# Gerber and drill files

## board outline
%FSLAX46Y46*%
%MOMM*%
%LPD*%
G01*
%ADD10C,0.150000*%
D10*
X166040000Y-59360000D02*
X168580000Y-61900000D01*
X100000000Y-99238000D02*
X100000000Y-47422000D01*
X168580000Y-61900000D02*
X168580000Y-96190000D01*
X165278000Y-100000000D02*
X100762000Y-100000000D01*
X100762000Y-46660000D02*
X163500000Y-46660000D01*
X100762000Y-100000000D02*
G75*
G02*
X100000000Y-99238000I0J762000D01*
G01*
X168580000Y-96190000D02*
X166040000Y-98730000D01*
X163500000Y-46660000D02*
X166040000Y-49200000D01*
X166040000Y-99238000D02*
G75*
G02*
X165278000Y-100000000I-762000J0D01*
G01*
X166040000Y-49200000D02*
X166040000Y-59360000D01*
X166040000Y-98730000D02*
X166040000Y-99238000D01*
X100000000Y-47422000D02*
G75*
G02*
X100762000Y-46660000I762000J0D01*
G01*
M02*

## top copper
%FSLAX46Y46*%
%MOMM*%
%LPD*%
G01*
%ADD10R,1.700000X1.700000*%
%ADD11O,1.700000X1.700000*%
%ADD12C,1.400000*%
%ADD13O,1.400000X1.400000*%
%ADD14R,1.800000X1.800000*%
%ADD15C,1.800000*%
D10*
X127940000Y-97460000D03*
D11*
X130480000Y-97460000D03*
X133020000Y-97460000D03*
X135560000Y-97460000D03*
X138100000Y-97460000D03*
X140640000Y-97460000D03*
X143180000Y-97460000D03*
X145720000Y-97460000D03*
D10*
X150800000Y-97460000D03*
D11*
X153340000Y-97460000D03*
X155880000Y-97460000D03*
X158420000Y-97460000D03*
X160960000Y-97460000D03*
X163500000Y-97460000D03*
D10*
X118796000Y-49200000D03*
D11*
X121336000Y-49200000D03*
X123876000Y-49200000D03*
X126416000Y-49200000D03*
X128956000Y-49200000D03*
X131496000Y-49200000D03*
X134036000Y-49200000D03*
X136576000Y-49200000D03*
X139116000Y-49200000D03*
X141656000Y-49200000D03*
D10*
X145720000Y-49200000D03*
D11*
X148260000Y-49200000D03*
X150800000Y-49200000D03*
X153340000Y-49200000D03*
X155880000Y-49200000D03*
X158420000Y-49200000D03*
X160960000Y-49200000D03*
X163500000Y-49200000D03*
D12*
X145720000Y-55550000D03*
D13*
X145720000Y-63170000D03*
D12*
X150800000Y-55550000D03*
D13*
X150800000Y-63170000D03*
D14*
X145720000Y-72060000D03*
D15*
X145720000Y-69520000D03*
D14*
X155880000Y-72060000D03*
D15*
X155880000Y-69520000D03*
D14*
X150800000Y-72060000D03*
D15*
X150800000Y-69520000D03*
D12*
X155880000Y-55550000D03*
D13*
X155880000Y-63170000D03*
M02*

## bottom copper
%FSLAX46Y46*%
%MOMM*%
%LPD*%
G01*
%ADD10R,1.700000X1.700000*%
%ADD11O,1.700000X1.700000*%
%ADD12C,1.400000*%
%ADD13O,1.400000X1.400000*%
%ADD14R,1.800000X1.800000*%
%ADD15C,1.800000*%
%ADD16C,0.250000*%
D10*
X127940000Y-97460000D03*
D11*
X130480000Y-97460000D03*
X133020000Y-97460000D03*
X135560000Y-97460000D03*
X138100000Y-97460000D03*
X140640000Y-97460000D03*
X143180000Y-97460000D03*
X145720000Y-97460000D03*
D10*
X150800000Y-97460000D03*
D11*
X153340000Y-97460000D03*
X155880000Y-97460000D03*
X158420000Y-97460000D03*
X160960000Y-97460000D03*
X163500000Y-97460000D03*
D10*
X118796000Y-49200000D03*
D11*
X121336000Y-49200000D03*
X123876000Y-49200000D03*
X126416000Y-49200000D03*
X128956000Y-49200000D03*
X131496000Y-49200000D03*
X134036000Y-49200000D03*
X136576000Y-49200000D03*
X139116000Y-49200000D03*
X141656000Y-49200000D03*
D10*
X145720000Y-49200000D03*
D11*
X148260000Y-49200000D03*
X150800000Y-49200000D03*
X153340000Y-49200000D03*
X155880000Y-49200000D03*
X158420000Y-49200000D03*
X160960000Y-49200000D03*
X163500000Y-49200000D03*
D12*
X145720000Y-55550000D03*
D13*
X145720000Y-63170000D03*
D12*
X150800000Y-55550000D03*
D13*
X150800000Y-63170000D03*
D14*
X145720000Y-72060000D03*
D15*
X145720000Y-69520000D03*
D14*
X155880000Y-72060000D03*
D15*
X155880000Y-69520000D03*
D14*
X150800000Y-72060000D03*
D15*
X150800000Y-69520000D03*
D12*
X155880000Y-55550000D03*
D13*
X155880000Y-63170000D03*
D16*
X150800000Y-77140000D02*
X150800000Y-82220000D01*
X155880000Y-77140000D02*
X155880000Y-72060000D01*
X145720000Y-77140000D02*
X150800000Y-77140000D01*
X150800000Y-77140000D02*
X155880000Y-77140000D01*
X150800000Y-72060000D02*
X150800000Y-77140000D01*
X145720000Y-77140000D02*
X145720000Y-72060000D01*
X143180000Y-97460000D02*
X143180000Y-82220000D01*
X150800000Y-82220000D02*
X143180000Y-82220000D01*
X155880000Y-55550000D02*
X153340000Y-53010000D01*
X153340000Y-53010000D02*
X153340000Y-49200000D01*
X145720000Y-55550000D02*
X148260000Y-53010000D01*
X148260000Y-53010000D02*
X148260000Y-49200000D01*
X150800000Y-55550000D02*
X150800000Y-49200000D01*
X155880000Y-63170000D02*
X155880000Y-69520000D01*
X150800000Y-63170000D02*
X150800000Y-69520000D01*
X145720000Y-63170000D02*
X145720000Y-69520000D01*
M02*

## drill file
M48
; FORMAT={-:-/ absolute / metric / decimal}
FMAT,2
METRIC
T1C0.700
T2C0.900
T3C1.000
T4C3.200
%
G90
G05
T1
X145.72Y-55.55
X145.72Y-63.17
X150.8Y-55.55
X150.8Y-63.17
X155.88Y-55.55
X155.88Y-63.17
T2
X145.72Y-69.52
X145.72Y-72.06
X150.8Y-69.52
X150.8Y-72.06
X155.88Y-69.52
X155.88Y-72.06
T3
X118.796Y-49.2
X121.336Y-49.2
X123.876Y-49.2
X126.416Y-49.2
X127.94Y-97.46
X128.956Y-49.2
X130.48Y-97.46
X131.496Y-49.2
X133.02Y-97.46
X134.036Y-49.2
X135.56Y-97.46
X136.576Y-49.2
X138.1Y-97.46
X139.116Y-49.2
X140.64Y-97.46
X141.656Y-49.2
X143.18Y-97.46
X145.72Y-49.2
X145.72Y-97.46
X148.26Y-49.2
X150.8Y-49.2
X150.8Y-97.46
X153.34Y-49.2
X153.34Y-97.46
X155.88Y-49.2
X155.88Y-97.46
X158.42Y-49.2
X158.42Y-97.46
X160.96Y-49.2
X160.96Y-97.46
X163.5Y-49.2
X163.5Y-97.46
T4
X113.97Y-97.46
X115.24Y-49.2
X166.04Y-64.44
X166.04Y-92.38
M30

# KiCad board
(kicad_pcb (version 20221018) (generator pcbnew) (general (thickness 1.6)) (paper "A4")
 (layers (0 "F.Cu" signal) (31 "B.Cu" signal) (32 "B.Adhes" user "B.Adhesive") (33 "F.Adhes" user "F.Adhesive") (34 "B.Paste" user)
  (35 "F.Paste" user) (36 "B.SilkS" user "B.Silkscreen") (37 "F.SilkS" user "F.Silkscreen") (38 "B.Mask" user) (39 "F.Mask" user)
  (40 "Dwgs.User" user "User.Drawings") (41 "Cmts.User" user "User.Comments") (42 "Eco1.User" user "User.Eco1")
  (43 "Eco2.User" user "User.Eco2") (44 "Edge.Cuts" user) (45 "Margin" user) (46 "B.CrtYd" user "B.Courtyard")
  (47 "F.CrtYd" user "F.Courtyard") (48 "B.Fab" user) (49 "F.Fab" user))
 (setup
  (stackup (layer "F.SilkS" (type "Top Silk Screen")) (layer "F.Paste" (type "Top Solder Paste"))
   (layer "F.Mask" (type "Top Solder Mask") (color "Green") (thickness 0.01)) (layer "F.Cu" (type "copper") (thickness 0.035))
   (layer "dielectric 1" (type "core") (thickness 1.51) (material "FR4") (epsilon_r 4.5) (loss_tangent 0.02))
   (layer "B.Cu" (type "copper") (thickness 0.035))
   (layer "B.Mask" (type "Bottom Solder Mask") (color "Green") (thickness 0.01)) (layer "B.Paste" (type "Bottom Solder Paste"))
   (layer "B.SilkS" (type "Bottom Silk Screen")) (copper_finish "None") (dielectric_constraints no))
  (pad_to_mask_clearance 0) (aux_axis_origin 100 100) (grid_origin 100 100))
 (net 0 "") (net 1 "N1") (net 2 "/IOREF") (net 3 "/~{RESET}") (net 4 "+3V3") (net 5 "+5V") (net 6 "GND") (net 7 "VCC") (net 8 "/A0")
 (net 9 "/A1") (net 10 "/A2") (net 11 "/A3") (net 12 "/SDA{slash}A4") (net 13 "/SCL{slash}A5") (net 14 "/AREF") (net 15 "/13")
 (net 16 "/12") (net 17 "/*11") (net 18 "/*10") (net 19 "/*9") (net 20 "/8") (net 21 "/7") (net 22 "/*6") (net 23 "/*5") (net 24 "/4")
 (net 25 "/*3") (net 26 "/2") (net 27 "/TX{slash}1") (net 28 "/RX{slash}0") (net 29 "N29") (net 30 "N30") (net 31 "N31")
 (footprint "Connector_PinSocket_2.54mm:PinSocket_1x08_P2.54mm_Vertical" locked (layer "F.Cu") (at 127.94 97.46 90)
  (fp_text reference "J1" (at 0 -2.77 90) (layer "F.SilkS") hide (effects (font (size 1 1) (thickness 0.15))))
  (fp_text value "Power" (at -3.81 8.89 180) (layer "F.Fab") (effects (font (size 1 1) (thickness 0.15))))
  (pad "1" thru_hole rect locked (at 0 0 90) (size 1.7 1.7) (drill 1) (layers "*.Cu" "*.Mask") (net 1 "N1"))
  (pad "2" thru_hole oval locked (at 0 2.54 90) (size 1.7 1.7) (drill 1) (layers "*.Cu" "*.Mask") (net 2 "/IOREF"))
  (pad "3" thru_hole oval locked (at 0 5.08 90) (size 1.7 1.7) (drill 1) (layers "*.Cu" "*.Mask") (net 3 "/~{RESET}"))
  (pad "4" thru_hole oval locked (at 0 7.62 90) (size 1.7 1.7) (drill 1) (layers "*.Cu" "*.Mask") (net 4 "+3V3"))
  (pad "5" thru_hole oval locked (at 0 10.16 90) (size 1.7 1.7) (drill 1) (layers "*.Cu" "*.Mask") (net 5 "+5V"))
  (pad "6" thru_hole oval locked (at 0 12.7 90) (size 1.7 1.7) (drill 1) (layers "*.Cu" "*.Mask") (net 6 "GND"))
  (pad "7" thru_hole oval locked (at 0 15.24 90) (size 1.7 1.7) (drill 1) (layers "*.Cu" "*.Mask") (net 6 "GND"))
  (pad "8" thru_hole oval locked (at 0 17.78 90) (size 1.7 1.7) (drill 1) (layers "*.Cu" "*.Mask") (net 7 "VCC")))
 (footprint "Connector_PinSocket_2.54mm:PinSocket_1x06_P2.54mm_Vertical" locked (layer "F.Cu") (at 150.8 97.46 90)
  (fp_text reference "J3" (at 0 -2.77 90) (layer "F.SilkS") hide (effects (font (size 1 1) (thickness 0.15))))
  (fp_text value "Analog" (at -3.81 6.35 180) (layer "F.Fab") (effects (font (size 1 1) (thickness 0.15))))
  (pad "1" thru_hole rect locked (at 0 0 90) (size 1.7 1.7) (drill 1) (layers "*.Cu" "*.Mask") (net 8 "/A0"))
  (pad "2" thru_hole oval locked (at 0 2.54 90) (size 1.7 1.7) (drill 1) (layers "*.Cu" "*.Mask") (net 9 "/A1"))
  (pad "3" thru_hole oval locked (at 0 5.08 90) (size 1.7 1.7) (drill 1) (layers "*.Cu" "*.Mask") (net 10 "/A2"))
  (pad "4" thru_hole oval locked (at 0 7.62 90) (size 1.7 1.7) (drill 1) (layers "*.Cu" "*.Mask") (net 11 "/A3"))
  (pad "5" thru_hole oval locked (at 0 10.16 90) (size 1.7 1.7) (drill 1) (layers "*.Cu" "*.Mask") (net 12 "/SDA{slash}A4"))
  (pad "6" thru_hole oval locked (at 0 12.7 90) (size 1.7 1.7) (drill 1) (layers "*.Cu" "*.Mask") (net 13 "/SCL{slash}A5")))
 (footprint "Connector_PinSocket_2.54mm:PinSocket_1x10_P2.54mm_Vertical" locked (layer "F.Cu") (at 118.796 49.2 90)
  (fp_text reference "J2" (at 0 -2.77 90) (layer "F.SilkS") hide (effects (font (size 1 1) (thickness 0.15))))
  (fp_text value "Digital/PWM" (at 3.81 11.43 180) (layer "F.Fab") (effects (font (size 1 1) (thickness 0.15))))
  (pad "1" thru_hole rect locked (at 0 0 90) (size 1.7 1.7) (drill 1) (layers "*.Cu" "*.Mask") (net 13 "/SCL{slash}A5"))
  (pad "2" thru_hole oval locked (at 0 2.54 90) (size 1.7 1.7) (drill 1) (layers "*.Cu" "*.Mask") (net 12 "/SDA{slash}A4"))
  (pad "3" thru_hole oval locked (at 0 5.08 90) (size 1.7 1.7) (drill 1) (layers "*.Cu" "*.Mask") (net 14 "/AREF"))
  (pad "4" thru_hole oval locked (at 0 7.62 90) (size 1.7 1.7) (drill 1) (layers "*.Cu" "*.Mask") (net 6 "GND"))
  (pad "5" thru_hole oval locked (at 0 10.16 90) (size 1.7 1.7) (drill 1) (layers "*.Cu" "*.Mask") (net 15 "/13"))
  (pad "6" thru_hole oval locked (at 0 12.7 90) (size 1.7 1.7) (drill 1) (layers "*.Cu" "*.Mask") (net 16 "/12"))
  (pad "7" thru_hole oval locked (at 0 15.24 90) (size 1.7 1.7) (drill 1) (layers "*.Cu" "*.Mask") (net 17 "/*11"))
  (pad "8" thru_hole oval locked (at 0 17.78 90) (size 1.7 1.7) (drill 1) (layers "*.Cu" "*.Mask") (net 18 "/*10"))
  (pad "9" thru_hole oval locked (at 0 20.32 90) (size 1.7 1.7) (drill 1) (layers "*.Cu" "*.Mask") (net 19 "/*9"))
  (pad "10" thru_hole oval locked (at 0 22.86 90) (size 1.7 1.7) (drill 1) (layers "*.Cu" "*.Mask") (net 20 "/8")))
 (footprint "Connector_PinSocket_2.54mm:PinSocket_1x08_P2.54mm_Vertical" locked (layer "F.Cu") (at 145.72 49.2 90)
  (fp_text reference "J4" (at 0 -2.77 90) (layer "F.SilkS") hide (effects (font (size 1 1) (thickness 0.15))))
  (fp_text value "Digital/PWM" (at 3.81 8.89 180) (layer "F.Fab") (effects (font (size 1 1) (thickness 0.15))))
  (pad "1" thru_hole rect locked (at 0 0 90) (size 1.7 1.7) (drill 1) (layers "*.Cu" "*.Mask") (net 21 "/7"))
  (pad "2" thru_hole oval locked (at 0 2.54 90) (size 1.7 1.7) (drill 1) (layers "*.Cu" "*.Mask") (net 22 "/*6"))
  (pad "3" thru_hole oval locked (at 0 5.08 90) (size 1.7 1.7) (drill 1) (layers "*.Cu" "*.Mask") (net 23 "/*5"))
  (pad "4" thru_hole oval locked (at 0 7.62 90) (size 1.7 1.7) (drill 1) (layers "*.Cu" "*.Mask") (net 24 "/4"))
  (pad "5" thru_hole oval locked (at 0 10.16 90) (size 1.7 1.7) (drill 1) (layers "*.Cu" "*.Mask") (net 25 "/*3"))
  (pad "6" thru_hole oval locked (at 0 12.7 90) (size 1.7 1.7) (drill 1) (layers "*.Cu" "*.Mask") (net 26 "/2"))
  (pad "7" thru_hole oval locked (at 0 15.24 90) (size 1.7 1.7) (drill 1) (layers "*.Cu" "*.Mask") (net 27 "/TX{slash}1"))
  (pad "8" thru_hole oval locked (at 0 17.78 90) (size 1.7 1.7) (drill 1) (layers "*.Cu" "*.Mask") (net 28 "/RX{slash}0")))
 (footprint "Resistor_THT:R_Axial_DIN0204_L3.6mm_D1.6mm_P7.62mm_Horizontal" (layer "F.Cu") (at 145.72 55.55 -90)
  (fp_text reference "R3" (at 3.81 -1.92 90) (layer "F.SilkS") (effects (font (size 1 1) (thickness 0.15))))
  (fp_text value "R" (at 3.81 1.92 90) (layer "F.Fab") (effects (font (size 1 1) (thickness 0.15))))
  (pad "1" thru_hole circle (at 0 0 270) (size 1.4 1.4) (drill 0.7) (layers "*.Cu" "*.Mask") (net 22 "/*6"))
  (pad "2" thru_hole oval (at 7.62 0 270) (size 1.4 1.4) (drill 0.7) (layers "*.Cu" "*.Mask") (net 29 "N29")))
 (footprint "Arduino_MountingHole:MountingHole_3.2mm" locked (layer "F.Cu") (at 115.24 49.2)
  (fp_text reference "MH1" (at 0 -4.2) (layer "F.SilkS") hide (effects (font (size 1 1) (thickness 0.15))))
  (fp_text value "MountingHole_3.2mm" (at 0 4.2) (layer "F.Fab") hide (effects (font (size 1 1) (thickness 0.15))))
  (pad "" np_thru_hole circle locked (at 0 0) (size 3.2 3.2) (drill 3.2) (layers "*.Cu" "*.Mask")))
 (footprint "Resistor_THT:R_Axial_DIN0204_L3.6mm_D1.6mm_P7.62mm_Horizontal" (layer "F.Cu") (at 150.8 55.55 -90)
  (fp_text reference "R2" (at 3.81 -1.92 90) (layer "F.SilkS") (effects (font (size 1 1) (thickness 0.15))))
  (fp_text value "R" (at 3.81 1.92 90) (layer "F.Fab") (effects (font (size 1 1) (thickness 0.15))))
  (pad "1" thru_hole circle (at 0 0 270) (size 1.4 1.4) (drill 0.7) (layers "*.Cu" "*.Mask") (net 23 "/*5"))
  (pad "2" thru_hole oval (at 7.62 0 270) (size 1.4 1.4) (drill 0.7) (layers "*.Cu" "*.Mask") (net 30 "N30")))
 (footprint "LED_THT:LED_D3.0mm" (layer "F.Cu") (at 145.72 72.06 90)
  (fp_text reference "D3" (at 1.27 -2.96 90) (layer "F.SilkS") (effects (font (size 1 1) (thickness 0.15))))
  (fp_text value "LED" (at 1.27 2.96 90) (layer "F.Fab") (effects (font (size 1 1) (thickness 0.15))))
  (pad "1" thru_hole rect (at 0 0 90) (size 1.8 1.8) (drill 0.9) (layers "*.Cu" "*.Mask") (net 6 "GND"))
  (pad "2" thru_hole circle (at 2.54 0 90) (size 1.8 1.8) (drill 0.9) (layers "*.Cu" "*.Mask") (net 29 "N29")))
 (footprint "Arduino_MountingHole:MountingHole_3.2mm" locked (layer "F.Cu") (at 113.97 97.46)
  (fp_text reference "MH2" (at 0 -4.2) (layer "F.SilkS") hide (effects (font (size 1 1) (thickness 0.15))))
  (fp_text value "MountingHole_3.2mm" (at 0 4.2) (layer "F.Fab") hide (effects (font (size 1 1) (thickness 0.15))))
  (pad "" np_thru_hole circle locked (at 0 0) (size 3.2 3.2) (drill 3.2) (layers "*.Cu" "*.Mask")))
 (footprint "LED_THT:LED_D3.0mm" (layer "F.Cu") (at 155.88 72.06 90)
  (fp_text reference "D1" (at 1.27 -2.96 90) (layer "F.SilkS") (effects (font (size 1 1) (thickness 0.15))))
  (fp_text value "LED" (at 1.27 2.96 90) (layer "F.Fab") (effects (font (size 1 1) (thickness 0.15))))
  (pad "1" thru_hole rect (at 0 0 90) (size 1.8 1.8) (drill 0.9) (layers "*.Cu" "*.Mask") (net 6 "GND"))
  (pad "2" thru_hole circle (at 2.54 0 90) (size 1.8 1.8) (drill 0.9) (layers "*.Cu" "*.Mask") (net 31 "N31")))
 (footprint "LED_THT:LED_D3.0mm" (layer "F.Cu") (at 150.8 72.06 90)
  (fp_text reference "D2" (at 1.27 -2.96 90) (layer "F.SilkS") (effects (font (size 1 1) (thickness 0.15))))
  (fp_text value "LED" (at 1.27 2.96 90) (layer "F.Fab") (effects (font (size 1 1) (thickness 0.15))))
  (pad "1" thru_hole rect (at 0 0 90) (size 1.8 1.8) (drill 0.9) (layers "*.Cu" "*.Mask") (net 6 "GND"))
  (pad "2" thru_hole circle (at 2.54 0 90) (size 1.8 1.8) (drill 0.9) (layers "*.Cu" "*.Mask") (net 30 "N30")))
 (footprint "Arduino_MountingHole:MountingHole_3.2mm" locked (layer "F.Cu") (at 166.04 64.44)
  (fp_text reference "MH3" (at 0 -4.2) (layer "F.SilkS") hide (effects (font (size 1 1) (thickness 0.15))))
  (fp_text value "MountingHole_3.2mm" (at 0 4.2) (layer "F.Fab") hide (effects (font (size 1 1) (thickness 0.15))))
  (pad "" np_thru_hole circle locked (at 0 0) (size 3.2 3.2) (drill 3.2) (layers "*.Cu" "*.Mask")))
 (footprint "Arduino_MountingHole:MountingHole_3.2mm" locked (layer "F.Cu") (at 166.04 92.38)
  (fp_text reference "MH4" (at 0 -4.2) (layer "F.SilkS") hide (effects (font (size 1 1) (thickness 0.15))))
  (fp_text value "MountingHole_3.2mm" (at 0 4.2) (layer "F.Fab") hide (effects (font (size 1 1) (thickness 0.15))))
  (pad "" np_thru_hole circle locked (at 0 0) (size 3.2 3.2) (drill 3.2) (layers "*.Cu" "*.Mask")))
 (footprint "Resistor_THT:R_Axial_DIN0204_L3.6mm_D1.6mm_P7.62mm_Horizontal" (layer "F.Cu") (at 155.88 55.55 -90)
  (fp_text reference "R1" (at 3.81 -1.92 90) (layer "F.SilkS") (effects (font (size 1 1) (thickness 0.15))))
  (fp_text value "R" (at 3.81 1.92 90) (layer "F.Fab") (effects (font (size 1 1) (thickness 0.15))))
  (pad "1" thru_hole circle (at 0 0 270) (size 1.4 1.4) (drill 0.7) (layers "*.Cu" "*.Mask") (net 24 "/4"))
  (pad "2" thru_hole oval (at 7.62 0 270) (size 1.4 1.4) (drill 0.7) (layers "*.Cu" "*.Mask") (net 31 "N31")))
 (gr_line (start 166.04 59.36) (end 168.58 61.9) (stroke (width 0.15) (type solid)) (layer "Edge.Cuts"))
 (gr_line (start 100 99.238) (end 100 47.422) (stroke (width 0.15) (type solid)) (layer "Edge.Cuts"))
 (gr_line (start 168.58 61.9) (end 168.58 96.19) (stroke (width 0.15) (type solid)) (layer "Edge.Cuts"))
 (gr_line (start 165.278 100) (end 100.762 100) (stroke (width 0.15) (type solid)) (layer "Edge.Cuts"))
 (gr_line (start 100.762 46.66) (end 163.5 46.66) (stroke (width 0.15) (type solid)) (layer "Edge.Cuts"))
 (gr_arc (start 100.762 100) (mid 100.223185 99.776815) (end 100 99.238) (stroke (width 0.15) (type solid)) (layer "Edge.Cuts"))
 (gr_line (start 168.58 96.19) (end 166.04 98.73) (stroke (width 0.15) (type solid)) (layer "Edge.Cuts"))
 (gr_line (start 163.5 46.66) (end 166.04 49.2) (stroke (width 0.15) (type solid)) (layer "Edge.Cuts"))
 (gr_arc (start 166.04 99.238) (mid 165.816815 99.776815) (end 165.278 100) (stroke (width 0.15) (type solid)) (layer "Edge.Cuts"))
 (gr_line (start 166.04 49.2) (end 166.04 59.36) (stroke (width 0.15) (type solid)) (layer "Edge.Cuts"))
 (gr_line (start 166.04 98.73) (end 166.04 99.238) (stroke (width 0.15) (type solid)) (layer "Edge.Cuts"))
 (gr_arc (start 100 47.422) (mid 100.223185 46.883185) (end 100.762 46.66) (stroke (width 0.15) (type solid)) (layer "Edge.Cuts"))
 (segment (start 150.8 77.14) (end 150.8 82.22) (width 0.25) (layer "B.Cu") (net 6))
 (segment (start 155.88 77.14) (end 155.88 72.06) (width 0.25) (layer "B.Cu") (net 6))
 (segment (start 145.72 77.14) (end 150.8 77.14) (width 0.25) (layer "B.Cu") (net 6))
 (segment (start 150.8 77.14) (end 155.88 77.14) (width 0.25) (layer "B.Cu") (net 6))
 (segment (start 150.8 72.06) (end 150.8 77.14) (width 0.25) (layer "B.Cu") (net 6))
 (segment (start 145.72 77.14) (end 145.72 72.06) (width 0.25) (layer "B.Cu") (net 6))
 (segment (start 143.18 97.46) (end 143.18 82.22) (width 0.25) (layer "B.Cu") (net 6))
 (segment (start 150.8 82.22) (end 143.18 82.22) (width 0.25) (layer "B.Cu") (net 6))
 (segment (start 155.88 55.55) (end 153.34 53.01) (width 0.25) (layer "B.Cu") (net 24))
 (segment (start 153.34 53.01) (end 153.34 49.2) (width 0.25) (layer "B.Cu") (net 24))
 (segment (start 145.72 55.55) (end 148.26 53.01) (width 0.25) (layer "B.Cu") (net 22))
 (segment (start 148.26 53.01) (end 148.26 49.2) (width 0.25) (layer "B.Cu") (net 22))
 (segment (start 150.8 55.55) (end 150.8 49.2) (width 0.25) (layer "B.Cu") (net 23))
 (segment (start 155.88 63.17) (end 155.88 69.52) (width 0.25) (layer "B.Cu") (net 31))
 (segment (start 150.8 63.17) (end 150.8 69.52) (width 0.25) (layer "B.Cu") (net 30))
 (segment (start 145.72 63.17) (end 145.72 69.52) (width 0.25) (layer "B.Cu") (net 29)))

